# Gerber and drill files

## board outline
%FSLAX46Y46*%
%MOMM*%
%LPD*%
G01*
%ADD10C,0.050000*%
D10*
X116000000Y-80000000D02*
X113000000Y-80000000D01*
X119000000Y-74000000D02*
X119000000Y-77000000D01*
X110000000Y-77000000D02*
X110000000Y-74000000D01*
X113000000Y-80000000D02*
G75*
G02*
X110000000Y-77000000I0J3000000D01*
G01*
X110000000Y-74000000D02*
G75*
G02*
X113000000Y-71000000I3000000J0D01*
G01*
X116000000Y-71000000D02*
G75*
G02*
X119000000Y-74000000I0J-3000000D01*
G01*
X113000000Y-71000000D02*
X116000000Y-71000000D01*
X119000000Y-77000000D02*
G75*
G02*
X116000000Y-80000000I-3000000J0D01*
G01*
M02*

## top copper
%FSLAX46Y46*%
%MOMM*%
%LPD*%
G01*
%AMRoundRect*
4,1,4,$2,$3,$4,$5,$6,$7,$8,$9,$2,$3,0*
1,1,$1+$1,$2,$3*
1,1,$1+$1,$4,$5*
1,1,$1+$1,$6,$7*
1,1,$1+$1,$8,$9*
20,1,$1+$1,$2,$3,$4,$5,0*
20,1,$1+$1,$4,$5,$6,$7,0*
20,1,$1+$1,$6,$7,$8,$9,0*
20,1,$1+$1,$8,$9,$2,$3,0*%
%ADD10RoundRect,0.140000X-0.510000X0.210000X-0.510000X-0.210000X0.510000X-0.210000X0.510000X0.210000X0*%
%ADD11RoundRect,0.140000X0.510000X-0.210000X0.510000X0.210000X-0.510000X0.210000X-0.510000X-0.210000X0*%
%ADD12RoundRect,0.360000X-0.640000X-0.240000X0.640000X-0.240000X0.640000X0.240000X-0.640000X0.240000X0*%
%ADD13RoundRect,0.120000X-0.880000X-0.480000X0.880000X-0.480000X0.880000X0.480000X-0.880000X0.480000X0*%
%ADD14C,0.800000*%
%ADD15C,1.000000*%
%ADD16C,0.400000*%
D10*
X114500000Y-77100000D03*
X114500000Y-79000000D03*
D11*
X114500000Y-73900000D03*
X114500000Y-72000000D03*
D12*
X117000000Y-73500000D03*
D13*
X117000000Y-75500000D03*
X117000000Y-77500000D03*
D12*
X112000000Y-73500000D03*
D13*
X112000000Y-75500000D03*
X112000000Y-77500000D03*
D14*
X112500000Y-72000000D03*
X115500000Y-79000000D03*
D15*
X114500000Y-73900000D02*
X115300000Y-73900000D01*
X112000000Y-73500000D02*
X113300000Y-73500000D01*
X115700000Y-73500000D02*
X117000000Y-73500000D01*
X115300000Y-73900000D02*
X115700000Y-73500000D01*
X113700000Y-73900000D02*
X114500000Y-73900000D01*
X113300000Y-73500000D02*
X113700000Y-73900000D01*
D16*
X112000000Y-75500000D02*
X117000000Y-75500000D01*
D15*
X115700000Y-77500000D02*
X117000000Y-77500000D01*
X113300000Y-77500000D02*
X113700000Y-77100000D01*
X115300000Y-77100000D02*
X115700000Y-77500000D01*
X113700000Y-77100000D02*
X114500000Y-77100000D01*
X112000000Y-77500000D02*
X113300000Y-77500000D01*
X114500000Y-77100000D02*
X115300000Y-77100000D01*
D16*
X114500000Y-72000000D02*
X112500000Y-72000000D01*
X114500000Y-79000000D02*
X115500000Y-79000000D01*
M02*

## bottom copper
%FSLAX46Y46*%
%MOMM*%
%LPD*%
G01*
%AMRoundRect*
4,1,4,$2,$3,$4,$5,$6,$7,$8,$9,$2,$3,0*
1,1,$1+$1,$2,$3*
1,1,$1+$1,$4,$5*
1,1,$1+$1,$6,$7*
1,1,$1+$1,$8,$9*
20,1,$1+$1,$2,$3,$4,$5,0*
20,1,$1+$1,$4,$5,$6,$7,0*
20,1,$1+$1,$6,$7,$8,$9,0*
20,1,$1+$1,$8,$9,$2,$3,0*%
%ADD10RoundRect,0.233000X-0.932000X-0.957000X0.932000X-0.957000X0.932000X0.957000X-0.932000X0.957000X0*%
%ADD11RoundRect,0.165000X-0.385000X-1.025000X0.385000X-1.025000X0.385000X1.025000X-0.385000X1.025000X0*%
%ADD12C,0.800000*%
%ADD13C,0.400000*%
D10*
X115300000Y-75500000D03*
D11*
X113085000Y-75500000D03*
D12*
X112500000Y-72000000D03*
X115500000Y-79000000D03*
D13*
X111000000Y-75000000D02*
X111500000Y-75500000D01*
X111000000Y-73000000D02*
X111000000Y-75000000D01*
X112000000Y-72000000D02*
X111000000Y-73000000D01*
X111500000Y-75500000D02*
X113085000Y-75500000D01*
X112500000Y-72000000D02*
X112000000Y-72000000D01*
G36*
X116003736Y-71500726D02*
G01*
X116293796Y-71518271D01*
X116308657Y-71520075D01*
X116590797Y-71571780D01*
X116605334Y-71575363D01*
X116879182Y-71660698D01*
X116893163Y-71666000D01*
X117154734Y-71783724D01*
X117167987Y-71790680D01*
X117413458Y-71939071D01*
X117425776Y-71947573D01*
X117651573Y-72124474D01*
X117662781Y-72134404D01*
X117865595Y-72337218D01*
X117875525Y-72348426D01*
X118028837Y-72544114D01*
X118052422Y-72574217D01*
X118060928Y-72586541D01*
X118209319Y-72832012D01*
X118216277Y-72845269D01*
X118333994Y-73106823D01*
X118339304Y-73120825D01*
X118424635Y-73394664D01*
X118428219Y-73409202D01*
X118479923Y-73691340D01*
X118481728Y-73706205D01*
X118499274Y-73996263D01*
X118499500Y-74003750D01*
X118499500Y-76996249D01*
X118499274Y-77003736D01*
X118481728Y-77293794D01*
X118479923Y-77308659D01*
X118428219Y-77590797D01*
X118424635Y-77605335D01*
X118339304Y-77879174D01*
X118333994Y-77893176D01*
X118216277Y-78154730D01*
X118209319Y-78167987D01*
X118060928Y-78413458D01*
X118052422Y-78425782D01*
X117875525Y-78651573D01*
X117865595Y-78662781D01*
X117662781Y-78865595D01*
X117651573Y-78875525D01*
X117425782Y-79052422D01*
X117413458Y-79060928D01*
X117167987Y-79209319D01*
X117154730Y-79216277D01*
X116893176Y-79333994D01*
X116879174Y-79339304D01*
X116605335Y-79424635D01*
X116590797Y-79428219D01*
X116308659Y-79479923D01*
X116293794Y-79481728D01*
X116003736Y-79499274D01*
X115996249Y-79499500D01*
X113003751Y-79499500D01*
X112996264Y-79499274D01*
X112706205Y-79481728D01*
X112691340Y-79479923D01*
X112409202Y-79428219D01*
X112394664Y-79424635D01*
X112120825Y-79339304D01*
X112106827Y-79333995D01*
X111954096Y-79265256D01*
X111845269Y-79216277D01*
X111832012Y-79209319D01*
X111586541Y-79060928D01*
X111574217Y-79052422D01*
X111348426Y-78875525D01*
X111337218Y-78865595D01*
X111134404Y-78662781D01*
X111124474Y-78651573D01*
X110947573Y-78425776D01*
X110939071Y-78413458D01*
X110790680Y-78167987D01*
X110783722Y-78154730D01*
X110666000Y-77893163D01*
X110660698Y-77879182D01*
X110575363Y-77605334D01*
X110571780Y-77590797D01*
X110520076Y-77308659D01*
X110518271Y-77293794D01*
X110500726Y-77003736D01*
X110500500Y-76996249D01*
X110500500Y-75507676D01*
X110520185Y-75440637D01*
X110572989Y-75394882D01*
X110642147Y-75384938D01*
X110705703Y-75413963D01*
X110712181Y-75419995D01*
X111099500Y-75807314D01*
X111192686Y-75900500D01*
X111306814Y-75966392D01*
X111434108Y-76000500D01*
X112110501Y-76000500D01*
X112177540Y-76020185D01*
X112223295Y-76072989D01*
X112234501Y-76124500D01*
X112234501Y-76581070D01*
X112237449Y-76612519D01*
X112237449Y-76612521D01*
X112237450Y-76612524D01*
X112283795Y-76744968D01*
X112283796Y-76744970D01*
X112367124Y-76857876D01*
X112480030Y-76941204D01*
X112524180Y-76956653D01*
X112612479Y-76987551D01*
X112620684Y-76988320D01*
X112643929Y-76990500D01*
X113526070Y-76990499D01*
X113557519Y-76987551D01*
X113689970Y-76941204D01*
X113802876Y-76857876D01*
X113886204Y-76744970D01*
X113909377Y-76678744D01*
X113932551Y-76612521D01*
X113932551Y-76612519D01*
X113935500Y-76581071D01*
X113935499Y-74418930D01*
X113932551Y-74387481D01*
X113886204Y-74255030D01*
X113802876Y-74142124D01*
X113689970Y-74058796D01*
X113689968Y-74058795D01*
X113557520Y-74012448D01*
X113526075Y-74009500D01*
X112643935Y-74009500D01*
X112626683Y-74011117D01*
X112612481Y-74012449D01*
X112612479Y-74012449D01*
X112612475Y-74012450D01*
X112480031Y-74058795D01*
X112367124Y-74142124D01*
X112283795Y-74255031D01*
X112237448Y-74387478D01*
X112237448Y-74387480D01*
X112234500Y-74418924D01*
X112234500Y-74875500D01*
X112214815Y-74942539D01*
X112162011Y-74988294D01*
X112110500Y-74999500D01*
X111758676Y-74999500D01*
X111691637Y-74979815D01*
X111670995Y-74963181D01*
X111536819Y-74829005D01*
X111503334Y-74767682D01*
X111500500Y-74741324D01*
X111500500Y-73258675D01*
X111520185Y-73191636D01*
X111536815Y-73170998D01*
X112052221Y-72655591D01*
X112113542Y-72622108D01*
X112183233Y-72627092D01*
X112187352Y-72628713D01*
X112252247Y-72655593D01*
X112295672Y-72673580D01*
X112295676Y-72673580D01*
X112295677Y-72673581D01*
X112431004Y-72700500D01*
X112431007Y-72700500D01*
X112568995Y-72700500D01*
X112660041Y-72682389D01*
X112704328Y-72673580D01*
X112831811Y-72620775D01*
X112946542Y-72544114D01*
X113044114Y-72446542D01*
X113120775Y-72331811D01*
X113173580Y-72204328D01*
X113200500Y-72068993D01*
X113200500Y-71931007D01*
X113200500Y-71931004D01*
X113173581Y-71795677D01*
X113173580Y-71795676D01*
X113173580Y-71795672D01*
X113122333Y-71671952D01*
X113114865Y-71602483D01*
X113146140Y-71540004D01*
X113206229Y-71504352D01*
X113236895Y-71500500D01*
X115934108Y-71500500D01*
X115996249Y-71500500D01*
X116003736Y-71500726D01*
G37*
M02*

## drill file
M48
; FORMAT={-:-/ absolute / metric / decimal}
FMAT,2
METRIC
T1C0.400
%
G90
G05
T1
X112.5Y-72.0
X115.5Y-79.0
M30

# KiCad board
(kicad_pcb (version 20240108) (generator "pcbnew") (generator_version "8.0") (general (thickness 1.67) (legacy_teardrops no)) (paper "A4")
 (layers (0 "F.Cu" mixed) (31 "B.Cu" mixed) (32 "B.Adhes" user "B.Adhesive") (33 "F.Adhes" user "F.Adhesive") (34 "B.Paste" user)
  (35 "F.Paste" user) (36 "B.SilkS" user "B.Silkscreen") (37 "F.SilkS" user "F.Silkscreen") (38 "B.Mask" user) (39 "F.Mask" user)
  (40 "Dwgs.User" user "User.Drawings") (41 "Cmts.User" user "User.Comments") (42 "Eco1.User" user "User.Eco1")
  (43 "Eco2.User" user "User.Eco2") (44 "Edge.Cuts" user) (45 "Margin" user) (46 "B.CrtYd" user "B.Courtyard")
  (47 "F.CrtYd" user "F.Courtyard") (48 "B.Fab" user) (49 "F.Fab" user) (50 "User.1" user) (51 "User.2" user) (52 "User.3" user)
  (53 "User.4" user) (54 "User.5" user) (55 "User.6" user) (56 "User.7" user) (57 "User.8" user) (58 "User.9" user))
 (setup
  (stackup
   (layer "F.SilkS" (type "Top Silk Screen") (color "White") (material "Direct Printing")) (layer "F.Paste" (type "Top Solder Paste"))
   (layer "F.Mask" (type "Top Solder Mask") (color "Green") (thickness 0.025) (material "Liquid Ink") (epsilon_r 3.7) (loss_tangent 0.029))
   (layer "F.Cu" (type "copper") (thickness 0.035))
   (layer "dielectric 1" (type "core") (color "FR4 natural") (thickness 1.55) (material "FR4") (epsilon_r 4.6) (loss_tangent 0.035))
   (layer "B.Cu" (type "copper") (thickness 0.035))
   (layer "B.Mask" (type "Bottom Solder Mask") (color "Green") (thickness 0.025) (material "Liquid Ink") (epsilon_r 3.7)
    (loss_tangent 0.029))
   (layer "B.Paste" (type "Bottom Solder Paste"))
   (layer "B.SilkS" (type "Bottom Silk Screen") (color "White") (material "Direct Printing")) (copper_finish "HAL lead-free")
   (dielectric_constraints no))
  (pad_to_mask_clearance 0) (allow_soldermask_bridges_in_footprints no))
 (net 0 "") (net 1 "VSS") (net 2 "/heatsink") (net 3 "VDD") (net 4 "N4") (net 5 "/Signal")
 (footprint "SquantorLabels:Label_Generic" (layer "F.Cu") (at 138.1 91.5)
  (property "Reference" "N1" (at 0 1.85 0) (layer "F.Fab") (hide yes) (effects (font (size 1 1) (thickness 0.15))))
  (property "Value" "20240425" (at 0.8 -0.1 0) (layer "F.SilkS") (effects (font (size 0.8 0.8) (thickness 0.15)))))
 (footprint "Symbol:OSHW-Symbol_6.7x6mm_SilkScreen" (layer "F.Cu") (at 138.7 87.6)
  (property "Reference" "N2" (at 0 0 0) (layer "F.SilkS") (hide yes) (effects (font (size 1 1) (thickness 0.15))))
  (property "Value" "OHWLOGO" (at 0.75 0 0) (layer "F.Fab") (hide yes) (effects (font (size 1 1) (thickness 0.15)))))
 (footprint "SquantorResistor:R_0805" (layer "F.Cu") (at 114.5 78.05 -90)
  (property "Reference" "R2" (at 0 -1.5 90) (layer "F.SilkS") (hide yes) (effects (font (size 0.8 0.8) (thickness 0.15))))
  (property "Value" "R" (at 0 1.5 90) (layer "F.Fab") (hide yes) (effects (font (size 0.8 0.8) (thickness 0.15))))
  (pad "1" smd roundrect (at -0.95 0 270) (size 0.7 1.3) (layers "F.Cu" "F.Paste" "F.Mask") (roundrect_rratio 0.2) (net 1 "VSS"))
  (pad "2" smd roundrect (at 0.95 0 270) (size 0.7 1.3) (layers "F.Cu" "F.Paste" "F.Mask") (roundrect_rratio 0.2) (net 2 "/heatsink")))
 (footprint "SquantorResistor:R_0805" (layer "F.Cu") (at 114.5 72.95 90)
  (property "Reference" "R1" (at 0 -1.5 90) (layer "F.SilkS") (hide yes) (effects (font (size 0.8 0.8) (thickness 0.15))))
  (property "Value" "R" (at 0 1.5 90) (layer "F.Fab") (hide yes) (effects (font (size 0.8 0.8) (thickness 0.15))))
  (pad "1" smd roundrect (at -0.95 0 90) (size 0.7 1.3) (layers "F.Cu" "F.Paste" "F.Mask") (roundrect_rratio 0.2) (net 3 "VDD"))
  (pad "2" smd roundrect (at 0.95 0 90) (size 0.7 1.3) (layers "F.Cu" "F.Paste" "F.Mask") (roundrect_rratio 0.2) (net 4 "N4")))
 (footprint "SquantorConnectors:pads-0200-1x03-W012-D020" (layer "F.Cu") (at 117 75.5)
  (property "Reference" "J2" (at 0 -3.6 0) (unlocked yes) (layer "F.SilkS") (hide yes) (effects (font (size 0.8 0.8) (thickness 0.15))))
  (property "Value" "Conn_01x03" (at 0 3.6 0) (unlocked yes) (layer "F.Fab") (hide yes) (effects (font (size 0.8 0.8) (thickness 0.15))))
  (pad "1" smd roundrect (at 0 -2) (size 2 1.2) (layers "F.Cu" "F.Paste" "F.Mask") (roundrect_rratio 0.3) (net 3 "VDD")
   (thermal_bridge_angle 45))
  (pad "2" smd roundrect (at 0 0) (size 2 1.2) (layers "F.Cu" "F.Paste" "F.Mask") (roundrect_rratio 0.1) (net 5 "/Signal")
   (thermal_bridge_angle 45))
  (pad "3" smd roundrect (at 0 2) (size 2 1.2) (layers "F.Cu" "F.Paste" "F.Mask") (roundrect_rratio 0.1) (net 1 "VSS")
   (thermal_bridge_angle 45)))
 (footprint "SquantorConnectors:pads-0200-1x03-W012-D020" (layer "F.Cu") (at 112 75.5)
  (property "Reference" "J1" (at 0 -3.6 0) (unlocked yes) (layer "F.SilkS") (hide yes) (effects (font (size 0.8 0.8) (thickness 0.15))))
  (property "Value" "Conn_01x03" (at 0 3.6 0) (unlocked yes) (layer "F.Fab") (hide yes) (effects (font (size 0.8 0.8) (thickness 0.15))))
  (pad "1" smd roundrect (at 0 -2) (size 2 1.2) (layers "F.Cu" "F.Paste" "F.Mask") (roundrect_rratio 0.3) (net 3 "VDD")
   (thermal_bridge_angle 45))
  (pad "2" smd roundrect (at 0 0) (size 2 1.2) (layers "F.Cu" "F.Paste" "F.Mask") (roundrect_rratio 0.1) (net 5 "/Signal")
   (thermal_bridge_angle 45))
  (pad "3" smd roundrect (at 0 2) (size 2 1.2) (layers "F.Cu" "F.Paste" "F.Mask") (roundrect_rratio 0.1) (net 1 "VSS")
   (thermal_bridge_angle 45)))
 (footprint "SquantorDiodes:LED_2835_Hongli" (layer "B.Cu") (at 114.5 75.5 180)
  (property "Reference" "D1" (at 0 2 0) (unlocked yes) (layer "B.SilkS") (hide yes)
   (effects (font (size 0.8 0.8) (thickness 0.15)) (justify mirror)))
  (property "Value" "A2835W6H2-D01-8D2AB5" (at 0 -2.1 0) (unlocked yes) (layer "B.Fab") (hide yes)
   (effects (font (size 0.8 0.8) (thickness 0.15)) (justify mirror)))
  (pad "1" smd roundrect (at -0.8 0) (size 2.33 2.38) (layers "B.Cu" "B.Paste" "B.Mask") (roundrect_rratio 0.1) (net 2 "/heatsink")
   (thermal_bridge_angle 45))
  (pad "2" smd roundrect (at 1.415 0) (size 1.1 2.38) (layers "B.Cu" "B.Paste" "B.Mask") (roundrect_rratio 0.15) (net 4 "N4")
   (thermal_bridge_angle 45)))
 (gr_line (start 116 80) (end 113 80) (stroke (width 0.05) (type default)) (layer "Edge.Cuts"))
 (gr_line (start 119 74) (end 119 77) (stroke (width 0.05) (type default)) (layer "Edge.Cuts"))
 (gr_line (start 110 77) (end 110 74) (stroke (width 0.05) (type default)) (layer "Edge.Cuts"))
 (gr_arc (start 113 80) (mid 110.87868 79.12132) (end 110 77) (stroke (width 0.05) (type default)) (layer "Edge.Cuts"))
 (gr_arc (start 110 74) (mid 110.87868 71.87868) (end 113 71) (stroke (width 0.05) (type default)) (layer "Edge.Cuts"))
 (gr_arc (start 116 71) (mid 118.12132 71.87868) (end 119 74) (stroke (width 0.05) (type default)) (layer "Edge.Cuts"))
 (gr_line (start 113 71) (end 116 71) (stroke (width 0.05) (type default)) (layer "Edge.Cuts"))
 (gr_arc (start 119 77) (mid 118.12132 79.12132) (end 116 80) (stroke (width 0.05) (type default)) (layer "Edge.Cuts"))
 (segment (start 114.5 73.9) (end 115.3 73.9) (width 1) (layer "F.Cu") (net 3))
 (segment (start 112 73.5) (end 113.3 73.5) (width 1) (layer "F.Cu") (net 3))
 (segment (start 115.7 73.5) (end 117 73.5) (width 1) (layer "F.Cu") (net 3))
 (segment (start 115.3 73.9) (end 115.7 73.5) (width 1) (layer "F.Cu") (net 3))
 (segment (start 113.7 73.9) (end 114.5 73.9) (width 1) (layer "F.Cu") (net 3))
 (segment (start 113.3 73.5) (end 113.7 73.9) (width 1) (layer "F.Cu") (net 3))
 (segment (start 112 75.5) (end 117 75.5) (width 0.4) (layer "F.Cu") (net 5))
 (segment (start 115.7 77.5) (end 117 77.5) (width 1) (layer "F.Cu") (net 1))
 (segment (start 113.3 77.5) (end 113.7 77.1) (width 1) (layer "F.Cu") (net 1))
 (segment (start 115.3 77.1) (end 115.7 77.5) (width 1) (layer "F.Cu") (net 1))
 (segment (start 113.7 77.1) (end 114.5 77.1) (width 1) (layer "F.Cu") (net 1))
 (segment (start 112 77.5) (end 113.3 77.5) (width 1) (layer "F.Cu") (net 1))
 (segment (start 114.5 77.1) (end 115.3 77.1) (width 1) (layer "F.Cu") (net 1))
 (segment (start 114.5 72) (end 112.5 72) (width 0.4) (layer "F.Cu") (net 4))
 (via (at 112.5 72) (size 0.8) (drill 0.4) (layers "F.Cu" "B.Cu") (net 4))
 (segment (start 111 75) (end 111.5 75.5) (width 0.4) (layer "B.Cu") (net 4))
 (segment (start 111 73) (end 111 75) (width 0.4) (layer "B.Cu") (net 4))
 (segment (start 112 72) (end 111 73) (width 0.4) (layer "B.Cu") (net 4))
 (segment (start 111.5 75.5) (end 113.085 75.5) (width 0.4) (layer "B.Cu") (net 4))
 (segment (start 112.5 72) (end 112 72) (width 0.4) (layer "B.Cu") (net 4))
 (segment (start 114.5 79) (end 115.5 79) (width 0.4) (layer "F.Cu") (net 2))
 (via (at 115.5 79) (size 0.8) (drill 0.4) (layers "F.Cu" "B.Cu") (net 2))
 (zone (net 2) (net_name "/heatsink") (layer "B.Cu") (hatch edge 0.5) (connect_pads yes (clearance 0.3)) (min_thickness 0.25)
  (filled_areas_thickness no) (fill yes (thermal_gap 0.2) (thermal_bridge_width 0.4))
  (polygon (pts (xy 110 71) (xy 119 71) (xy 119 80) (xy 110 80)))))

